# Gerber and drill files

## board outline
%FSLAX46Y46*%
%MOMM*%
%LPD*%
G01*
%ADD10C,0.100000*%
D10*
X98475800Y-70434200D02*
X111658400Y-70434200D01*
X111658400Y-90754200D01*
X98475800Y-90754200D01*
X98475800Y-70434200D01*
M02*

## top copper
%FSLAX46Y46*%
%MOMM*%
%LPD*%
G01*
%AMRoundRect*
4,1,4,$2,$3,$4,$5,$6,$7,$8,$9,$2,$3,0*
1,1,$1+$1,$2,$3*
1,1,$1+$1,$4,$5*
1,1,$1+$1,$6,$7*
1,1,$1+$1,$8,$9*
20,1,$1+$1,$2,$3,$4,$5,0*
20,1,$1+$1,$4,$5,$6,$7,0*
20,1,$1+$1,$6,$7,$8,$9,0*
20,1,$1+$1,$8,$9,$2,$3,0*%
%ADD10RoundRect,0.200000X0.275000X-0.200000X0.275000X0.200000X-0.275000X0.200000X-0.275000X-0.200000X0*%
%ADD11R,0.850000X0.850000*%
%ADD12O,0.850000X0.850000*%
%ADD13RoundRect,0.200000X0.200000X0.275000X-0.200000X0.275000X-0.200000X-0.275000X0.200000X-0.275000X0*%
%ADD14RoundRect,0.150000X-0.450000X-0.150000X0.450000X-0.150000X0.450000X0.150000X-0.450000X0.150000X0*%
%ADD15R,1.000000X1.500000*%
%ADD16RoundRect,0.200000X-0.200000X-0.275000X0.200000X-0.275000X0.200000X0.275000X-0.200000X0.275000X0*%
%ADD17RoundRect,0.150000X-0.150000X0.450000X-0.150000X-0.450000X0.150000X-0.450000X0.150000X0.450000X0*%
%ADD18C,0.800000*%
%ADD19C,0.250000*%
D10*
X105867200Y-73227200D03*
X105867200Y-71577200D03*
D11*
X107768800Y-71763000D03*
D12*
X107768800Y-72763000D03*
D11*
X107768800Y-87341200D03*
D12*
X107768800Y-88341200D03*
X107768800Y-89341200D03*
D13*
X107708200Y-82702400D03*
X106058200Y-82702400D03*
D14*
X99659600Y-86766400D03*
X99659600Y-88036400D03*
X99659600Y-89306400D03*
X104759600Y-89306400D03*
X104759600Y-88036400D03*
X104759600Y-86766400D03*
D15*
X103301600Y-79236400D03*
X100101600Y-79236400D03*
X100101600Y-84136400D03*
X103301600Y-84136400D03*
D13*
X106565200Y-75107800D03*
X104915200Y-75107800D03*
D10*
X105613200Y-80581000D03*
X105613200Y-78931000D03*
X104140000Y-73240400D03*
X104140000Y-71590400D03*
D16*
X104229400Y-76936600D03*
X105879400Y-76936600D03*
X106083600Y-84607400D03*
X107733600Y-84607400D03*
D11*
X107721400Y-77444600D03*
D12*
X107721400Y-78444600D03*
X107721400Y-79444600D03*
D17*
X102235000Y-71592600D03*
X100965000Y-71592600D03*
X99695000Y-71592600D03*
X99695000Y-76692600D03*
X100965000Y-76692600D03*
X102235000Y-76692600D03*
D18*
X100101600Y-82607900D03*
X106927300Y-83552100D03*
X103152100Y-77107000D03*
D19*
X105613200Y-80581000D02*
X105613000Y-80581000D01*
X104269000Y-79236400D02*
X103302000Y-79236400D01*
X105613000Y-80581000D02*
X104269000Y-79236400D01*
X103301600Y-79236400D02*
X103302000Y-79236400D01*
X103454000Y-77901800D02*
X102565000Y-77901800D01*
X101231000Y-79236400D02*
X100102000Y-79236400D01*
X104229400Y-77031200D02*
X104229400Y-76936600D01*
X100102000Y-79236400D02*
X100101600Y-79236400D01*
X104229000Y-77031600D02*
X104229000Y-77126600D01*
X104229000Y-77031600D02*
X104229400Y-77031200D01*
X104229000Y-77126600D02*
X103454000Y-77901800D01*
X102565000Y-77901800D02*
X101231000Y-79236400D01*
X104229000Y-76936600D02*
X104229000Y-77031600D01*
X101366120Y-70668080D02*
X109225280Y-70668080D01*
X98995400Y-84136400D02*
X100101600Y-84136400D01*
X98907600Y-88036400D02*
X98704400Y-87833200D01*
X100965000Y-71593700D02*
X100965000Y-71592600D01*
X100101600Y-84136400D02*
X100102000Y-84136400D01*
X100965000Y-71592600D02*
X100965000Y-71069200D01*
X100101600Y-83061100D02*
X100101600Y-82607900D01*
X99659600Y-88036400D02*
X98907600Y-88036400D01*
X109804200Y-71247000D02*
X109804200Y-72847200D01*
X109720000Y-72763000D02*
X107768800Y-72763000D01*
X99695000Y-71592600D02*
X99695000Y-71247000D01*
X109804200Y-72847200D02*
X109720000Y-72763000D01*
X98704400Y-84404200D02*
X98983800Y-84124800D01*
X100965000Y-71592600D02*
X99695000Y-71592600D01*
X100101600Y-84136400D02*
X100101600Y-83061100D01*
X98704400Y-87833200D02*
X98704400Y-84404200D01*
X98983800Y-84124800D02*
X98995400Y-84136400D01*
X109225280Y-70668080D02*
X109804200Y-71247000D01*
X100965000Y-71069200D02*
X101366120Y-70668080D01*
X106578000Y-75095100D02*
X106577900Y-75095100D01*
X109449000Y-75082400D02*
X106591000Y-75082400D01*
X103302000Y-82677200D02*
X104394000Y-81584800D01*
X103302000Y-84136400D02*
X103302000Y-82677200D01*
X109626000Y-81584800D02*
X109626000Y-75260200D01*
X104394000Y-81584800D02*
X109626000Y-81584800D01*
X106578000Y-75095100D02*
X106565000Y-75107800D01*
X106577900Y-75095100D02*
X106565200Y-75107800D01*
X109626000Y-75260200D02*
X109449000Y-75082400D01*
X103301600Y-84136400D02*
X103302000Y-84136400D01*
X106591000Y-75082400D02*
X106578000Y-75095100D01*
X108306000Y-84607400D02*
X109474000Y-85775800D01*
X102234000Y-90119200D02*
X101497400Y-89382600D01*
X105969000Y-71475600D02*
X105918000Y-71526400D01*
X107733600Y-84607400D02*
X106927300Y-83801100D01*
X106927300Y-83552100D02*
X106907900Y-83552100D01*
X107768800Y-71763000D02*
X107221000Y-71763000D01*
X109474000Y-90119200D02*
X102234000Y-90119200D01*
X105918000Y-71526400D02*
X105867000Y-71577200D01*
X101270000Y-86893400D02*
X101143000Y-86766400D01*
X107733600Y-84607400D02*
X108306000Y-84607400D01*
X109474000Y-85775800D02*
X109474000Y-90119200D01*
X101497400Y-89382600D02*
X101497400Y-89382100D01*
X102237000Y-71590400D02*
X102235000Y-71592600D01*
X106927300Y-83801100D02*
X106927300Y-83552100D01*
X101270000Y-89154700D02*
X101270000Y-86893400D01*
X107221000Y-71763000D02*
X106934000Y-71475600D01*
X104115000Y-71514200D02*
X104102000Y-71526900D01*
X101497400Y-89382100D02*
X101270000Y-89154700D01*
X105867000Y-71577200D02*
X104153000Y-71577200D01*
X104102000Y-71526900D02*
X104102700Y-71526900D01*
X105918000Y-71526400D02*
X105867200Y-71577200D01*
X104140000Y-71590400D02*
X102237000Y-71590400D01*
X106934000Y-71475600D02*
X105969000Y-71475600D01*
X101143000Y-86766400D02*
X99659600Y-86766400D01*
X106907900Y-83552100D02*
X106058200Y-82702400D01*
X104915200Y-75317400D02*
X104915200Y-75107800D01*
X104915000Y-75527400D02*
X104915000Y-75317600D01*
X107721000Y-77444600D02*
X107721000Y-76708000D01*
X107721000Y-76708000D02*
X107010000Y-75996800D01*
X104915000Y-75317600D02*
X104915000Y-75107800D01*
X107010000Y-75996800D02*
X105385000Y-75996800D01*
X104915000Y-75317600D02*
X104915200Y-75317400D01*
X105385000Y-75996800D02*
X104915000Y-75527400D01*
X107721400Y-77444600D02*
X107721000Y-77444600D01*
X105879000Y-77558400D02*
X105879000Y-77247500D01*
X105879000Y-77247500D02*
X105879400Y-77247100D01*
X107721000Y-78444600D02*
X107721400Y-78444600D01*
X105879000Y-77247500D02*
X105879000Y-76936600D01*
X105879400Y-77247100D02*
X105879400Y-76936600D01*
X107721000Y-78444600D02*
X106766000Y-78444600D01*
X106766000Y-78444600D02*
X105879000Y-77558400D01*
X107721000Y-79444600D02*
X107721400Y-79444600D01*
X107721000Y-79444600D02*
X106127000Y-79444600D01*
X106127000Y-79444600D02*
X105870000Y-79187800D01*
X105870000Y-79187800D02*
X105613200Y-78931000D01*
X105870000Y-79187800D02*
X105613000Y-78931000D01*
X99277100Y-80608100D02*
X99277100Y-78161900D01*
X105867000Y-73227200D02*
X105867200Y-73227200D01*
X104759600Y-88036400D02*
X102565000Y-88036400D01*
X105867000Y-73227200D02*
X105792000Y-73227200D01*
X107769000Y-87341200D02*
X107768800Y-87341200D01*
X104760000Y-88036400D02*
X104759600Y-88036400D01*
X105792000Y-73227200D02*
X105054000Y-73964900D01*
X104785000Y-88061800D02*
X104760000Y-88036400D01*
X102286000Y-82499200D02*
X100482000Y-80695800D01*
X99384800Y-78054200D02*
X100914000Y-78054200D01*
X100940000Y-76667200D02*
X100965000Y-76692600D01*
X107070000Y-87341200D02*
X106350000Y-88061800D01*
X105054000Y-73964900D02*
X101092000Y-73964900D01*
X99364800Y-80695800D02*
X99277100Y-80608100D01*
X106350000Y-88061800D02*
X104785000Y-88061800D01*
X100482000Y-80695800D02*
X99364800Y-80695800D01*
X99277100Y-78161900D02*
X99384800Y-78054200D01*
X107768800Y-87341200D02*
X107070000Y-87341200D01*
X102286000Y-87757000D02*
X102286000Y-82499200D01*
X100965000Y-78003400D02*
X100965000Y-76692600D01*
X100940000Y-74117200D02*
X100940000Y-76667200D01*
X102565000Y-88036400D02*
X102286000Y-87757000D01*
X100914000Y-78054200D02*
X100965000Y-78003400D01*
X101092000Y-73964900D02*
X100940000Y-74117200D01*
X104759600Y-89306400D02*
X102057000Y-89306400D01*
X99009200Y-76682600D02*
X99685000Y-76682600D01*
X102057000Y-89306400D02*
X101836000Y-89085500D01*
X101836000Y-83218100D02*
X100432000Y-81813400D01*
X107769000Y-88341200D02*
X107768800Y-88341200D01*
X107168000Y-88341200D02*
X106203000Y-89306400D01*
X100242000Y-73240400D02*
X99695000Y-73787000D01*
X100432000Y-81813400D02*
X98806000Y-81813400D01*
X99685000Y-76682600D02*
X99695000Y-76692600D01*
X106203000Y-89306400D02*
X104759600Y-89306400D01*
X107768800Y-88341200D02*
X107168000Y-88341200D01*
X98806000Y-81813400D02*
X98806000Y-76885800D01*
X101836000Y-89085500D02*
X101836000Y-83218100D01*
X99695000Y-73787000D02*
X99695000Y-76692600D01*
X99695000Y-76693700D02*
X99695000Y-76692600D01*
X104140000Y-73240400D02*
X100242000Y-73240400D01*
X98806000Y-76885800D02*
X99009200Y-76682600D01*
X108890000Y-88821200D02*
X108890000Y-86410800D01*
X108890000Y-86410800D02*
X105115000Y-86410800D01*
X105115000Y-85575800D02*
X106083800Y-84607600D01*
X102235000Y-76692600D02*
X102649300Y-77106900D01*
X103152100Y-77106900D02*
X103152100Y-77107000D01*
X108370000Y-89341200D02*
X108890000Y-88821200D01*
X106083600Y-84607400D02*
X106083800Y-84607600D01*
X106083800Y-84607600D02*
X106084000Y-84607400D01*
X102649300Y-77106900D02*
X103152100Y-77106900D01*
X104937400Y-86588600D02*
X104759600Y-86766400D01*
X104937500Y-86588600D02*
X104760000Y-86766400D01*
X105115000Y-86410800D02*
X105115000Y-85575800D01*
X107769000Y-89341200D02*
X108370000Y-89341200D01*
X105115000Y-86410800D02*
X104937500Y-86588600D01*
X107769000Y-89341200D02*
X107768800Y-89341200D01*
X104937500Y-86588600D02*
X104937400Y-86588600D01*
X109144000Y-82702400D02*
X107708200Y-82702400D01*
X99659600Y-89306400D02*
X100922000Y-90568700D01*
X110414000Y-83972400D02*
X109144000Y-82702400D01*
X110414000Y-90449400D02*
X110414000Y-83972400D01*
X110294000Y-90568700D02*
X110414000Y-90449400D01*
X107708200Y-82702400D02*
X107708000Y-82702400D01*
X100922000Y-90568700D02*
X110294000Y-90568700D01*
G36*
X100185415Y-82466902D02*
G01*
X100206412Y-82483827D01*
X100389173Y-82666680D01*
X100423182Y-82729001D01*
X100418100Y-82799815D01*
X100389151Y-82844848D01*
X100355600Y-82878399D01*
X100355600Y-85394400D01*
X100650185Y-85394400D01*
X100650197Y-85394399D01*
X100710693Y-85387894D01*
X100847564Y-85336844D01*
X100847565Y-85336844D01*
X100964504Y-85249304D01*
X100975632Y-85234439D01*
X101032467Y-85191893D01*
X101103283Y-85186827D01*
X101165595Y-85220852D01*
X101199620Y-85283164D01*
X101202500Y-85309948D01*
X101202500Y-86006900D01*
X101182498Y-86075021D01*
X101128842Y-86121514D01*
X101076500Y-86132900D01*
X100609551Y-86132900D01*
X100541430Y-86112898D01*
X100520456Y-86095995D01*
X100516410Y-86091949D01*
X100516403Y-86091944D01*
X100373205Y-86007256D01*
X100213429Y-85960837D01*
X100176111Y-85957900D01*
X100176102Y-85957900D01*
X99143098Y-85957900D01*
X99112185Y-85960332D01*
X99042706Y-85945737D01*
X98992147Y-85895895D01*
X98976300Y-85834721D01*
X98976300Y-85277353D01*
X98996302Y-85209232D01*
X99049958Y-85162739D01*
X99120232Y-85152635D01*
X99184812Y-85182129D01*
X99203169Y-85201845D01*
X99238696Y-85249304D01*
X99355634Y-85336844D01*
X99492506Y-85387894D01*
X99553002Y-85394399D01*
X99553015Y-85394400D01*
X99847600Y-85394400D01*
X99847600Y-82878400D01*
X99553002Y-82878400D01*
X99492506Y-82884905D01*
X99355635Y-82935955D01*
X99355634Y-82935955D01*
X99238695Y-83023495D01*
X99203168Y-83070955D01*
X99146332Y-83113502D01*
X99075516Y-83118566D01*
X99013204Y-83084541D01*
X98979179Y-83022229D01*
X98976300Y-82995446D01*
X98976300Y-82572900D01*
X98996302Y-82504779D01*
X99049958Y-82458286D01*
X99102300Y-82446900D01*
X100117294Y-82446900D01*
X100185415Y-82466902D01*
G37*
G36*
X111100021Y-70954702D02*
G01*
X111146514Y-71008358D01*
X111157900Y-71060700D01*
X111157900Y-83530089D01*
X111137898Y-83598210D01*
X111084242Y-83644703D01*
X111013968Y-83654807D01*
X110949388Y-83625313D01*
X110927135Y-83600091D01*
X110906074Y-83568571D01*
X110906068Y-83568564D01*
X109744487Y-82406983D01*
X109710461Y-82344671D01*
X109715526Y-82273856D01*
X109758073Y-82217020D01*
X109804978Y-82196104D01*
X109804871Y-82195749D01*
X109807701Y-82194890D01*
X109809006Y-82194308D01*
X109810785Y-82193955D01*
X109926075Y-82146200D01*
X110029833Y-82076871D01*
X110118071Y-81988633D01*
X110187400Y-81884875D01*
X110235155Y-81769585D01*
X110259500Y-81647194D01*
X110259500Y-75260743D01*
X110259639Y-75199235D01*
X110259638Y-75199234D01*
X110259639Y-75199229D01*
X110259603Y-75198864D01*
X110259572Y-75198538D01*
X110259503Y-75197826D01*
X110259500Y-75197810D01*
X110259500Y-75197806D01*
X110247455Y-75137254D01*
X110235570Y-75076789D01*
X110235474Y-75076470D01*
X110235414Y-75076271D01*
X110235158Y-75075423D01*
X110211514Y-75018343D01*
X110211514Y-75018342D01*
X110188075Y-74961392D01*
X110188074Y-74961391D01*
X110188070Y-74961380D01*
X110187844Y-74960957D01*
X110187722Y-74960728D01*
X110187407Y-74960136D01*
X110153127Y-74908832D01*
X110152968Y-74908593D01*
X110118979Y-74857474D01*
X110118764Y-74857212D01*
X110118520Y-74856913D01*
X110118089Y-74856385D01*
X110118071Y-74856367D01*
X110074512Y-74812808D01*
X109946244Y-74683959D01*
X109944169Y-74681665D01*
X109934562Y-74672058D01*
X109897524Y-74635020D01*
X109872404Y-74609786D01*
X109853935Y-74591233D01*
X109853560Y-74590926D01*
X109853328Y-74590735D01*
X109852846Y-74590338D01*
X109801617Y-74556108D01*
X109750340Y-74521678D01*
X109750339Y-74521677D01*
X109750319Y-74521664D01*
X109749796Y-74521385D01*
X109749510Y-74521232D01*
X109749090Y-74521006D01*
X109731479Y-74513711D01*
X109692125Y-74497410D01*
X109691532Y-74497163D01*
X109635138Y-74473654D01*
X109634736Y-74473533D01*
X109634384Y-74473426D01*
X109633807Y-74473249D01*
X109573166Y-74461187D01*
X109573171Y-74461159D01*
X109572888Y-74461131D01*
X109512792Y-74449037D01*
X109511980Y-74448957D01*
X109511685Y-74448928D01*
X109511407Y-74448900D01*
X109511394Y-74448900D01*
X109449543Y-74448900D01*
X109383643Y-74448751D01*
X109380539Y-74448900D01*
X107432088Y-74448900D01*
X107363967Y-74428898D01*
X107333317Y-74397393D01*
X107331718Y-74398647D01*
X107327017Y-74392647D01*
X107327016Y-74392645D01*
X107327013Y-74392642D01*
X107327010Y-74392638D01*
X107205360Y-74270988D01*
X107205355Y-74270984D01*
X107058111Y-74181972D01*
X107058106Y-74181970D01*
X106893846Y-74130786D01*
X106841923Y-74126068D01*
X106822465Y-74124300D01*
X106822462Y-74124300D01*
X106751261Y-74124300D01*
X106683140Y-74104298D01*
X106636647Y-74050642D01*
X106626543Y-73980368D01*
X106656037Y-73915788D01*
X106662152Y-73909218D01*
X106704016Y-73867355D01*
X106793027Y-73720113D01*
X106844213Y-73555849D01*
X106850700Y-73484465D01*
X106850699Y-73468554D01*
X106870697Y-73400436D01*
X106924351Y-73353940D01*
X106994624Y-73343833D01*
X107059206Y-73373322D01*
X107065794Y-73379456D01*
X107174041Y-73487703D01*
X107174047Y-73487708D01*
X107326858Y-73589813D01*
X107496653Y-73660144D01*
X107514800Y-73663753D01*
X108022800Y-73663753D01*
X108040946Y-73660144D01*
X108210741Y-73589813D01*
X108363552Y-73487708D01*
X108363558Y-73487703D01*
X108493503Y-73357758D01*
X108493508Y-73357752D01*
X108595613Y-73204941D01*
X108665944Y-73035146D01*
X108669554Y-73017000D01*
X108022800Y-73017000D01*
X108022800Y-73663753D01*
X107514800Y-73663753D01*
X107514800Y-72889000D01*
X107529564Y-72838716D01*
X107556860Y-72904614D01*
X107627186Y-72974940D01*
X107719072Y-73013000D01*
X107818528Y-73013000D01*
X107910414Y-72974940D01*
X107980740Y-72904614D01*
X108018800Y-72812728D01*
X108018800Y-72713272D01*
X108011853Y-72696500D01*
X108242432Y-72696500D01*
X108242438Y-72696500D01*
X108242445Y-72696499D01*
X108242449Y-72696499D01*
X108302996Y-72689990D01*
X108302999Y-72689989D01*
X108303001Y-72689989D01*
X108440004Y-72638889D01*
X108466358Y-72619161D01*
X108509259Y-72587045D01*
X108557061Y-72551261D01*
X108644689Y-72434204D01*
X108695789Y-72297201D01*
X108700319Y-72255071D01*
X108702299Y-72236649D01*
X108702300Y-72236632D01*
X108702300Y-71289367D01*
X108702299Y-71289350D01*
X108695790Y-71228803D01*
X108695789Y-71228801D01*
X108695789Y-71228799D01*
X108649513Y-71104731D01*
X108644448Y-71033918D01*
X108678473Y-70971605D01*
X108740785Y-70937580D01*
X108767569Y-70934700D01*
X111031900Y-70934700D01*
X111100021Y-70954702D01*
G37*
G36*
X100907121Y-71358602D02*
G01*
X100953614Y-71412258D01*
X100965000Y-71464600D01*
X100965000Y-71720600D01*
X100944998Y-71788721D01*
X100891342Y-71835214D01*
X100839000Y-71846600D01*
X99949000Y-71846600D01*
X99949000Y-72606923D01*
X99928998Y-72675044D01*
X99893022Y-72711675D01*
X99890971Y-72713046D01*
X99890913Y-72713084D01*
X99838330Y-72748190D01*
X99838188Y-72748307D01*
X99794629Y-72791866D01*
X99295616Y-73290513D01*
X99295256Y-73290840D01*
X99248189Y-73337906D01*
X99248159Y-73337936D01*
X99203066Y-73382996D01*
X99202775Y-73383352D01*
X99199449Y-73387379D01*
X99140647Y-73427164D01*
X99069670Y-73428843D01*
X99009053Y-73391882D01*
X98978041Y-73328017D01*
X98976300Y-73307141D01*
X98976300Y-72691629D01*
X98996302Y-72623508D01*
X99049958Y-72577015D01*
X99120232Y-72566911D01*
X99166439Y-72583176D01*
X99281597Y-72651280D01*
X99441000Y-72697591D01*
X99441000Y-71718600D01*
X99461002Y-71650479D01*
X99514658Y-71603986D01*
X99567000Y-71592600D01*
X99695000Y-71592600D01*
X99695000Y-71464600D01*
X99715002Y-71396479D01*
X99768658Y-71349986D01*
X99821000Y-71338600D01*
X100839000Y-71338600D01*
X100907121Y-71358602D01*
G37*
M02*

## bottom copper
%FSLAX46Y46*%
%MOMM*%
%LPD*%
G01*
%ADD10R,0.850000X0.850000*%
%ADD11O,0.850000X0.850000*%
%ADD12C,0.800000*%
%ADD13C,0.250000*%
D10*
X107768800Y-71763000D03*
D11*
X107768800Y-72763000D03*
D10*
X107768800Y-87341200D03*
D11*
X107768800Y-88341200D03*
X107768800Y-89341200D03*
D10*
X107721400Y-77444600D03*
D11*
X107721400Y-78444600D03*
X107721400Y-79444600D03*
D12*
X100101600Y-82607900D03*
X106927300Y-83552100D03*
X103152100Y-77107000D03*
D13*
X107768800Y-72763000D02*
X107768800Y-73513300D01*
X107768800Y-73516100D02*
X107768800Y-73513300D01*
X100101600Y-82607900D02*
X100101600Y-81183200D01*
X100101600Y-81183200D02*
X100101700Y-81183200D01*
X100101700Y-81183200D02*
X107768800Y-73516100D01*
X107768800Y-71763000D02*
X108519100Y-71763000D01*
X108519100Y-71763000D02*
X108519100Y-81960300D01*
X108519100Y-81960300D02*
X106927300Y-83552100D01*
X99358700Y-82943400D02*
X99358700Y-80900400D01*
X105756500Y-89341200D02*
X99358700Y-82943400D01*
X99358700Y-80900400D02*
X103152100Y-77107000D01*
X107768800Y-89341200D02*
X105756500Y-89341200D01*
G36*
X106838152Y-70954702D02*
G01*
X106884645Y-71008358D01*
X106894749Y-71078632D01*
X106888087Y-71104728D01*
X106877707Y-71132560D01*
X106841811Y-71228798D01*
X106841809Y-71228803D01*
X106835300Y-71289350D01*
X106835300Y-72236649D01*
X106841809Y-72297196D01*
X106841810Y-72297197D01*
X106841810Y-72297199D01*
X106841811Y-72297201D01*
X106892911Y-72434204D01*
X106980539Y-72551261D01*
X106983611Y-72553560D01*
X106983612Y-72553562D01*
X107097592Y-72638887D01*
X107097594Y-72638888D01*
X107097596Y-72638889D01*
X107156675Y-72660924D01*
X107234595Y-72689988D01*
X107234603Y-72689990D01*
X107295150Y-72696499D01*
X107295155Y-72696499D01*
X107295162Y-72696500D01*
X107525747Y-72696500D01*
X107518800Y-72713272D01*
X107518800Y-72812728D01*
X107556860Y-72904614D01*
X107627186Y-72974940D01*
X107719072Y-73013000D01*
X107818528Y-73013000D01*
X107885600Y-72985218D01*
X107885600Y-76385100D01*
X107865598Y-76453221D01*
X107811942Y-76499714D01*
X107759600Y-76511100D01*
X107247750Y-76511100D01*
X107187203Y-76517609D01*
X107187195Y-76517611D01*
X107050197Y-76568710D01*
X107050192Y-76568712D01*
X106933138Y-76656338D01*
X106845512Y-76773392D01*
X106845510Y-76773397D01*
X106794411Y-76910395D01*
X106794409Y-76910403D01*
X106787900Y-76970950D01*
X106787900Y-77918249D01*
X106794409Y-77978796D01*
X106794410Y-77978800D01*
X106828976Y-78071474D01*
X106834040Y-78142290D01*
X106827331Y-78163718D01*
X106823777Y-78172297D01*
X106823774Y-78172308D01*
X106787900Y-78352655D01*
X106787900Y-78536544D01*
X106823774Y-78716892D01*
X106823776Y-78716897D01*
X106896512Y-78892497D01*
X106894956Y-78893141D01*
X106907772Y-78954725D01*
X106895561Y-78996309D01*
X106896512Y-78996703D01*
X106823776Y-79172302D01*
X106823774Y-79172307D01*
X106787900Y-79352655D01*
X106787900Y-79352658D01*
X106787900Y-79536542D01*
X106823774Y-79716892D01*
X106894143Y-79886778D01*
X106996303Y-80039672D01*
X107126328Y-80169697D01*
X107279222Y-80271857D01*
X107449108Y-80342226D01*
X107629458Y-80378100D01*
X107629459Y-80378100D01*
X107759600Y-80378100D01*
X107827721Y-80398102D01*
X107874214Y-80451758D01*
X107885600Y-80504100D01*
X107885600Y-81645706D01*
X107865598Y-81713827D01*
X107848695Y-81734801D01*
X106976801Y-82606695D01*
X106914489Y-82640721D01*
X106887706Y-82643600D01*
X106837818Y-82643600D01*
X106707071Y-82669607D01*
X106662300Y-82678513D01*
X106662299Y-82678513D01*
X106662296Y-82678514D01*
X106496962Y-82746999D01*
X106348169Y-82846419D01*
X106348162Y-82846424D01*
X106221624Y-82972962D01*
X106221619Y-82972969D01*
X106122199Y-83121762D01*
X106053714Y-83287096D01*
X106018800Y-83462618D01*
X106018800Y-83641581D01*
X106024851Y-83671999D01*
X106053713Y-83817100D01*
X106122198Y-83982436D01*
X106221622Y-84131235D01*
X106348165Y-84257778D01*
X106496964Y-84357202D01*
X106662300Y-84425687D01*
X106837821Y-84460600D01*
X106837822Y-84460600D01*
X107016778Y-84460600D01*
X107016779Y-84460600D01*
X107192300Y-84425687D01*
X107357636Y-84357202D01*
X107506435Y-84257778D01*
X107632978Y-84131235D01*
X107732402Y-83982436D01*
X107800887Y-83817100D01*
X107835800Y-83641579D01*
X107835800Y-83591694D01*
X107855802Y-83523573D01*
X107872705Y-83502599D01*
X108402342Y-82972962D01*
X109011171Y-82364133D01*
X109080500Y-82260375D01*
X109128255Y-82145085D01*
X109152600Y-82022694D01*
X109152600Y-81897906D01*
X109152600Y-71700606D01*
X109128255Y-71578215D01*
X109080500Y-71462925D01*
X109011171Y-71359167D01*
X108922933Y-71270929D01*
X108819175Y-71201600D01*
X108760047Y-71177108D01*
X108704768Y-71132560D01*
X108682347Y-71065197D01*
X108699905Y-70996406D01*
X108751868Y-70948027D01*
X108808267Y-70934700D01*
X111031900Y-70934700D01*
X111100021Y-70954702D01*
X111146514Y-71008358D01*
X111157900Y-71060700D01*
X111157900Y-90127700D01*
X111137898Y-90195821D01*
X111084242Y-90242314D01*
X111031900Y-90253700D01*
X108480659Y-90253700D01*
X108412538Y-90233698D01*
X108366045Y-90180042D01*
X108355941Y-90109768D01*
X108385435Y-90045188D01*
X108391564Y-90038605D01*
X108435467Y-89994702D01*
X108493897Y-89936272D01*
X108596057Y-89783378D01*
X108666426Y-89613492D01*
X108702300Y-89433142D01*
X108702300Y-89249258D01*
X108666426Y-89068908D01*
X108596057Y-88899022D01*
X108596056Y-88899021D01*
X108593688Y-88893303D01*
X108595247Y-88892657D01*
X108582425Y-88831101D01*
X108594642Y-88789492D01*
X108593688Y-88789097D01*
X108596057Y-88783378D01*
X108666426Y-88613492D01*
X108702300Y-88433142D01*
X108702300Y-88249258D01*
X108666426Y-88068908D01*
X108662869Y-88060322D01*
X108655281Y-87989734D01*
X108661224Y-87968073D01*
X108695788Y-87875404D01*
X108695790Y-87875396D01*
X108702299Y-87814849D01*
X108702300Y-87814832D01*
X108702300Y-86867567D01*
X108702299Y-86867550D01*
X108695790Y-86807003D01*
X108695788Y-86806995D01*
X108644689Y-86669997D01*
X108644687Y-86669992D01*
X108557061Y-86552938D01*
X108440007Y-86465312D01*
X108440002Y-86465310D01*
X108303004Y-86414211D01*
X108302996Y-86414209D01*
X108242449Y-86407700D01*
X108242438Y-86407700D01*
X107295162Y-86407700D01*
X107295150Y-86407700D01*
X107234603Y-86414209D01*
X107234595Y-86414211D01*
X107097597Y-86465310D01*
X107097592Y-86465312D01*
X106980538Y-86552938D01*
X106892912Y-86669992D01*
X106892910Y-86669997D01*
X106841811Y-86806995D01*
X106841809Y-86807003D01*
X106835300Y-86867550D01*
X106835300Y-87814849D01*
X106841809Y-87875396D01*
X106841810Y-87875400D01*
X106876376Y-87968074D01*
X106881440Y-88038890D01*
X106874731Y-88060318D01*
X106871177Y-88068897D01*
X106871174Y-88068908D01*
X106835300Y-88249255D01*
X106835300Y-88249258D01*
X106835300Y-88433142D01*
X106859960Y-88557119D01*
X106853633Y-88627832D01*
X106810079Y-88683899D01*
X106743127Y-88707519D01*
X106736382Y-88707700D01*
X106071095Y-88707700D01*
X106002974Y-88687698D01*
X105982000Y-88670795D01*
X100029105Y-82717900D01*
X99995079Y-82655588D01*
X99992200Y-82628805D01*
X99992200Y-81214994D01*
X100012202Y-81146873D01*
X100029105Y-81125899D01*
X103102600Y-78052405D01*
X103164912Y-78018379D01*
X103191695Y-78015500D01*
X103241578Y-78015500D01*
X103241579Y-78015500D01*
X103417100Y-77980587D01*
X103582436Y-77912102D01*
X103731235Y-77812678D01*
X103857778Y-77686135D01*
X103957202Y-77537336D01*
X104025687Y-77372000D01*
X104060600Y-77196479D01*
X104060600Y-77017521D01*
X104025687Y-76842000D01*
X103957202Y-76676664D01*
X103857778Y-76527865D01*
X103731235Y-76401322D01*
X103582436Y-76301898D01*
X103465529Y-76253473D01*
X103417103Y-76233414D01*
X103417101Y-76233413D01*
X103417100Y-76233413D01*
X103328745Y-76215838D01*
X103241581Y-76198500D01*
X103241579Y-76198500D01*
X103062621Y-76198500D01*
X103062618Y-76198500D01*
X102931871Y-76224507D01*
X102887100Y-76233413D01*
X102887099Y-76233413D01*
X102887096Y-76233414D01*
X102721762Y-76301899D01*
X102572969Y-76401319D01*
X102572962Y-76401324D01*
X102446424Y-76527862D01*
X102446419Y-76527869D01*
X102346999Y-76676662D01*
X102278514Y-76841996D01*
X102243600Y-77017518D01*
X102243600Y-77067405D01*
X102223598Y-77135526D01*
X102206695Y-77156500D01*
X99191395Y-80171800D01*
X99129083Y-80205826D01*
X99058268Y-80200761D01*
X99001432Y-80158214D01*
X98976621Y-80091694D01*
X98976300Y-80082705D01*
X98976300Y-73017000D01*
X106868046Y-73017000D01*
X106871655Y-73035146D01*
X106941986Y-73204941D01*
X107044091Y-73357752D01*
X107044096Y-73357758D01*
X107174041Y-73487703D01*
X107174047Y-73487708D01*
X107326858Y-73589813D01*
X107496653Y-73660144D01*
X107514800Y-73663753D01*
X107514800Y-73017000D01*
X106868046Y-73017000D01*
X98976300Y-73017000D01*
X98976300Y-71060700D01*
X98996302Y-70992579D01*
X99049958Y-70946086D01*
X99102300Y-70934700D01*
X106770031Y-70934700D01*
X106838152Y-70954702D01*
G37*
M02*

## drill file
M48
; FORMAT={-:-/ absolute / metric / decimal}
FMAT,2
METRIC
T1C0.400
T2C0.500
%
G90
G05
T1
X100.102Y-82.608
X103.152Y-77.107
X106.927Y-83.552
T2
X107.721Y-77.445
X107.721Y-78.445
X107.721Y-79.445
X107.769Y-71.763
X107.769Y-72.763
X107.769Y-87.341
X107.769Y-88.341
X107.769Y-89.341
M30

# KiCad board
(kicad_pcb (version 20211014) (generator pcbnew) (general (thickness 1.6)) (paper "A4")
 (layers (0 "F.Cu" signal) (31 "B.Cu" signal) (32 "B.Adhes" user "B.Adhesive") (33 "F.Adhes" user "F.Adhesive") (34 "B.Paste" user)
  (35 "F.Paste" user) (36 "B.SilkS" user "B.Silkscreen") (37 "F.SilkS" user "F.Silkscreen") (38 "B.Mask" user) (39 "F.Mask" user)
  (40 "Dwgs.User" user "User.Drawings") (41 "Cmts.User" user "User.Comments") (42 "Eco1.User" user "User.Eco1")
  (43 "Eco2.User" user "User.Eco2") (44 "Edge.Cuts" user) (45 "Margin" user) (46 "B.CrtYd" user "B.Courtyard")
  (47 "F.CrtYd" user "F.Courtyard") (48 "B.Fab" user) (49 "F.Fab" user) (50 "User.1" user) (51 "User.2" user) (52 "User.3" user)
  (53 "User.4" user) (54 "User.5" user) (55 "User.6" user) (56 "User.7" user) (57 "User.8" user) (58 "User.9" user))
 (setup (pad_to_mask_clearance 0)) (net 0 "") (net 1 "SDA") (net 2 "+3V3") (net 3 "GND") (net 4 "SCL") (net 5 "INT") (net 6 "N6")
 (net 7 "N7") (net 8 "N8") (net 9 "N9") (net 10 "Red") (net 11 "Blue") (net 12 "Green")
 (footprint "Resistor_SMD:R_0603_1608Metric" (layer "F.Cu") (at 105.8672 72.4022 90)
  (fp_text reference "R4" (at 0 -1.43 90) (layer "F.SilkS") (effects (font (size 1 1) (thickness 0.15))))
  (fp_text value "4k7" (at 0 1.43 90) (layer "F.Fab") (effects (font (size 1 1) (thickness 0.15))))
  (pad "1" smd roundrect (at -0.825 0 90) (size 0.8 0.95) (layers "F.Cu" "F.Paste" "F.Mask") (roundrect_rratio 0.25) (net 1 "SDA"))
  (pad "2" smd roundrect (at 0.825 0 90) (size 0.8 0.95) (layers "F.Cu" "F.Paste" "F.Mask") (roundrect_rratio 0.25) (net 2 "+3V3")))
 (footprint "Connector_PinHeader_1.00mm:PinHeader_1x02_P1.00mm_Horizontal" (layer "F.Cu") (at 107.7688 71.763)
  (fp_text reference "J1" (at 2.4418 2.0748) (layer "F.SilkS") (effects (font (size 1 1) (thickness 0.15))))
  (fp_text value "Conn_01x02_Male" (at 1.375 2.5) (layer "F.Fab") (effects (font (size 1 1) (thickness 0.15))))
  (pad "1" thru_hole rect (at 0 0) (size 0.85 0.85) (drill 0.5) (layers *.Cu *.Mask) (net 2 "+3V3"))
  (pad "2" thru_hole oval (at 0 1) (size 0.85 0.85) (drill 0.5) (layers *.Cu *.Mask) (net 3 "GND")))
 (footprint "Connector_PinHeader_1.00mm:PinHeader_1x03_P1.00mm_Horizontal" (layer "F.Cu") (at 107.7688 87.3412)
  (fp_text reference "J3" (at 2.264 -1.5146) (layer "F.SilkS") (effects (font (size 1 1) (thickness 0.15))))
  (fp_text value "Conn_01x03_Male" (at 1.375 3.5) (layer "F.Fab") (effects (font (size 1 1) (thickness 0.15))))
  (pad "1" thru_hole rect (at 0 0) (size 0.85 0.85) (drill 0.5) (layers *.Cu *.Mask) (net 1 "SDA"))
  (pad "2" thru_hole oval (at 0 1) (size 0.85 0.85) (drill 0.5) (layers *.Cu *.Mask) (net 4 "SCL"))
  (pad "3" thru_hole oval (at 0 2) (size 0.85 0.85) (drill 0.5) (layers *.Cu *.Mask) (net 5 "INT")))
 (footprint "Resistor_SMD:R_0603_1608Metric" (layer "F.Cu") (at 106.8832 82.7024 180)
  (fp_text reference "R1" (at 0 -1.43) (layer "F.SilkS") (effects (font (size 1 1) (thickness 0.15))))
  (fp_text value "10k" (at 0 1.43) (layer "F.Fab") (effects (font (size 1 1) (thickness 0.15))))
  (pad "1" smd roundrect (at -0.825 0 180) (size 0.8 0.95) (layers "F.Cu" "F.Paste" "F.Mask") (roundrect_rratio 0.25) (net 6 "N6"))
  (pad "2" smd roundrect (at 0.825 0 180) (size 0.8 0.95) (layers "F.Cu" "F.Paste" "F.Mask") (roundrect_rratio 0.25) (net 2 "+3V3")))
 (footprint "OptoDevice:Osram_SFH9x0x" (layer "F.Cu") (at 102.2096 88.0364)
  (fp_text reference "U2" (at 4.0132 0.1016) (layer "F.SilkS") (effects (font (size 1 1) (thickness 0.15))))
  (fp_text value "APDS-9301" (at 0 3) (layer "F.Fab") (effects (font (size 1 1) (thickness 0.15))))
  (pad "1" smd roundrect (at -2.55 -1.27) (size 1.2 0.6) (layers "F.Cu" "F.Paste" "F.Mask") (roundrect_rratio 0.25) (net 2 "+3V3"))
  (pad "2" smd roundrect (at -2.55 0) (size 1.2 0.6) (layers "F.Cu" "F.Paste" "F.Mask") (roundrect_rratio 0.25) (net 3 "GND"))
  (pad "3" smd roundrect (at -2.55 1.27) (size 1.2 0.6) (layers "F.Cu" "F.Paste" "F.Mask") (roundrect_rratio 0.25) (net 6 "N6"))
  (pad "4" smd roundrect (at 2.55 1.27) (size 1.2 0.6) (layers "F.Cu" "F.Paste" "F.Mask") (roundrect_rratio 0.25) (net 4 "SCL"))
  (pad "5" smd roundrect (at 2.55 0) (size 1.2 0.6) (layers "F.Cu" "F.Paste" "F.Mask") (roundrect_rratio 0.25) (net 1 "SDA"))
  (pad "6" smd roundrect (at 2.55 -1.27) (size 1.2 0.6) (layers "F.Cu" "F.Paste" "F.Mask") (roundrect_rratio 0.25) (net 5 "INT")))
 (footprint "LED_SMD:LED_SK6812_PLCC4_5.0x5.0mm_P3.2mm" (layer "F.Cu") (at 101.7016 81.6864 90)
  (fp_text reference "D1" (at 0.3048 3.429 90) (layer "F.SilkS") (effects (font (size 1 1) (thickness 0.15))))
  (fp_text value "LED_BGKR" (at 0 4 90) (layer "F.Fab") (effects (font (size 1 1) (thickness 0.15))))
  (pad "1" smd rect (at 2.45 1.6 90) (size 1.5 1) (layers "F.Cu" "F.Paste" "F.Mask") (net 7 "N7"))
  (pad "2" smd rect (at 2.45 -1.6 90) (size 1.5 1) (layers "F.Cu" "F.Paste" "F.Mask") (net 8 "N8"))
  (pad "3" smd rect (at -2.45 -1.6 90) (size 1.5 1) (layers "F.Cu" "F.Paste" "F.Mask") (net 3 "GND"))
  (pad "4" smd rect (at -2.45 1.6 90) (size 1.5 1) (layers "F.Cu" "F.Paste" "F.Mask") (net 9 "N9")))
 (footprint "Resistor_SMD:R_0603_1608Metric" (layer "F.Cu") (at 105.7402 75.1078 180)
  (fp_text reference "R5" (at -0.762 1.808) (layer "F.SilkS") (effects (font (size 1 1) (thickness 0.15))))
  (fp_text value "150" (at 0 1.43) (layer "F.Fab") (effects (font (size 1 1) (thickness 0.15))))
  (pad "1" smd roundrect (at -0.825 0 180) (size 0.8 0.95) (layers "F.Cu" "F.Paste" "F.Mask") (roundrect_rratio 0.25) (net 9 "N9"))
  (pad "2" smd roundrect (at 0.825 0 180) (size 0.8 0.95) (layers "F.Cu" "F.Paste" "F.Mask") (roundrect_rratio 0.25) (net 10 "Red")))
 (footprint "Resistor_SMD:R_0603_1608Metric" (layer "F.Cu") (at 105.6132 79.756 90)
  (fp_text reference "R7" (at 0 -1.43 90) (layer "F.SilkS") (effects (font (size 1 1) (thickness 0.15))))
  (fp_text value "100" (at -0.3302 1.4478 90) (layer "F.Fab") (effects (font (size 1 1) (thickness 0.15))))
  (pad "1" smd roundrect (at -0.825 0 90) (size 0.8 0.95) (layers "F.Cu" "F.Paste" "F.Mask") (roundrect_rratio 0.25) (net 7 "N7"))
  (pad "2" smd roundrect (at 0.825 0 90) (size 0.8 0.95) (layers "F.Cu" "F.Paste" "F.Mask") (roundrect_rratio 0.25) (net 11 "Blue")))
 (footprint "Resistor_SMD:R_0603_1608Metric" (layer "F.Cu") (at 104.14 72.4154 90)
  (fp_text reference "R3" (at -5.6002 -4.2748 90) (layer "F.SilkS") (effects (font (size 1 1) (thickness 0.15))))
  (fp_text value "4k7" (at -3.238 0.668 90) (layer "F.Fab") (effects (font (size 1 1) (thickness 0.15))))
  (pad "1" smd roundrect (at -0.825 0 90) (size 0.8 0.95) (layers "F.Cu" "F.Paste" "F.Mask") (roundrect_rratio 0.25) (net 4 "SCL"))
  (pad "2" smd roundrect (at 0.825 0 90) (size 0.8 0.95) (layers "F.Cu" "F.Paste" "F.Mask") (roundrect_rratio 0.25) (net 2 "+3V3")))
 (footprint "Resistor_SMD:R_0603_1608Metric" (layer "F.Cu") (at 105.0544 76.9366)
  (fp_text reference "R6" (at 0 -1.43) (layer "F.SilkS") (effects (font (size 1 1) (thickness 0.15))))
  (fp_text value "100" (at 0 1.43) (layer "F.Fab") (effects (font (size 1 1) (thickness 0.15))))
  (pad "1" smd roundrect (at -0.825 0) (size 0.8 0.95) (layers "F.Cu" "F.Paste" "F.Mask") (roundrect_rratio 0.25) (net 8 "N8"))
  (pad "2" smd roundrect (at 0.825 0) (size 0.8 0.95) (layers "F.Cu" "F.Paste" "F.Mask") (roundrect_rratio 0.25) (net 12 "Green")))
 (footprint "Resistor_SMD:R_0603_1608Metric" (layer "F.Cu") (at 106.9086 84.6074)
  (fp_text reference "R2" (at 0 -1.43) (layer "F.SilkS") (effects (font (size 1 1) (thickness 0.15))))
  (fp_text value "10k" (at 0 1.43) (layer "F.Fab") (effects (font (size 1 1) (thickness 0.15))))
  (pad "1" smd roundrect (at -0.825 0) (size 0.8 0.95) (layers "F.Cu" "F.Paste" "F.Mask") (roundrect_rratio 0.25) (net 5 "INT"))
  (pad "2" smd roundrect (at 0.825 0) (size 0.8 0.95) (layers "F.Cu" "F.Paste" "F.Mask") (roundrect_rratio 0.25) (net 2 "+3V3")))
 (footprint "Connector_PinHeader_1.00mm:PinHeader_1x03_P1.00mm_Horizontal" (layer "F.Cu") (at 107.7214 77.4446)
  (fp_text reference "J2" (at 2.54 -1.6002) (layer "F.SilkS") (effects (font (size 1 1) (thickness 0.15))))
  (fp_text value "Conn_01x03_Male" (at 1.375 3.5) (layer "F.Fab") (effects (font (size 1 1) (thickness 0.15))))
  (pad "1" thru_hole rect (at 0 0) (size 0.85 0.85) (drill 0.5) (layers *.Cu *.Mask) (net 10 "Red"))
  (pad "2" thru_hole oval (at 0 1) (size 0.85 0.85) (drill 0.5) (layers *.Cu *.Mask) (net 12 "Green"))
  (pad "3" thru_hole oval (at 0 2) (size 0.85 0.85) (drill 0.5) (layers *.Cu *.Mask) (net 11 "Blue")))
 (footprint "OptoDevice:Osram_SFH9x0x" (layer "F.Cu") (at 100.965 74.1426 -90)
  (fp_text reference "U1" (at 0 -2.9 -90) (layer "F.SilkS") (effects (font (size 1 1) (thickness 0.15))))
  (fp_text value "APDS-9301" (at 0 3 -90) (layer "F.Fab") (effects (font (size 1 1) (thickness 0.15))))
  (pad "1" smd roundrect (at -2.55 -1.27 270) (size 1.2 0.6) (layers "F.Cu" "F.Paste" "F.Mask") (roundrect_rratio 0.25) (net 2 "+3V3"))
  (pad "2" smd roundrect (at -2.55 0 270) (size 1.2 0.6) (layers "F.Cu" "F.Paste" "F.Mask") (roundrect_rratio 0.25) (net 3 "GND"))
  (pad "3" smd roundrect (at -2.55 1.27 270) (size 1.2 0.6) (layers "F.Cu" "F.Paste" "F.Mask") (roundrect_rratio 0.25) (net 3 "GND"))
  (pad "4" smd roundrect (at 2.55 1.27 270) (size 1.2 0.6) (layers "F.Cu" "F.Paste" "F.Mask") (roundrect_rratio 0.25) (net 4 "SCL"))
  (pad "5" smd roundrect (at 2.55 0 270) (size 1.2 0.6) (layers "F.Cu" "F.Paste" "F.Mask") (roundrect_rratio 0.25) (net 1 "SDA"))
  (pad "6" smd roundrect (at 2.55 -1.27 270) (size 1.2 0.6) (layers "F.Cu" "F.Paste" "F.Mask") (roundrect_rratio 0.25) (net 5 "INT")))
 (gr_rect (start 98.4758 70.4342) (end 111.6584 90.7542) (layer "Edge.Cuts") (width 0.1) (fill none))
 (segment (start 105.6132 80.581) (end 105.613 80.581) (width 0.25) (layer "F.Cu") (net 7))
 (segment (start 104.269 79.2364) (end 103.302 79.2364) (width 0.25) (layer "F.Cu") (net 7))
 (segment (start 105.613 80.581) (end 104.269 79.2364) (width 0.25) (layer "F.Cu") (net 7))
 (segment (start 103.3016 79.2364) (end 103.302 79.2364) (width 0.25) (layer "F.Cu") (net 7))
 (segment (start 103.454 77.9018) (end 102.565 77.9018) (width 0.25) (layer "F.Cu") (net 8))
 (segment (start 101.231 79.2364) (end 100.102 79.2364) (width 0.25) (layer "F.Cu") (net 8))
 (segment (start 104.2294 77.0312) (end 104.2294 76.9366) (width 0.25) (layer "F.Cu") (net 8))
 (segment (start 100.102 79.2364) (end 100.1016 79.2364) (width 0.25) (layer "F.Cu") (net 8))
 (segment (start 104.229 77.0316) (end 104.229 77.1266) (width 0.25) (layer "F.Cu") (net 8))
 (segment (start 104.229 77.0316) (end 104.2294 77.0312) (width 0.25) (layer "F.Cu") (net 8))
 (segment (start 104.229 77.1266) (end 103.454 77.9018) (width 0.25) (layer "F.Cu") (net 8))
 (segment (start 102.565 77.9018) (end 101.231 79.2364) (width 0.25) (layer "F.Cu") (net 8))
 (segment (start 104.229 76.9366) (end 104.229 77.0316) (width 0.25) (layer "F.Cu") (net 8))
 (segment (start 101.36612 70.66808) (end 109.22528 70.66808) (width 0.25) (layer "F.Cu") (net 3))
 (segment (start 98.9954 84.1364) (end 100.1016 84.1364) (width 0.25) (layer "F.Cu") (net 3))
 (segment (start 98.9076 88.0364) (end 98.7044 87.8332) (width 0.25) (layer "F.Cu") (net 3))
 (segment (start 100.965 71.5937) (end 100.965 71.5926) (width 0.25) (layer "F.Cu") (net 3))
 (segment (start 100.1016 84.1364) (end 100.102 84.1364) (width 0.25) (layer "F.Cu") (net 3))
 (segment (start 100.965 71.5926) (end 100.965 71.0692) (width 0.25) (layer "F.Cu") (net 3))
 (segment (start 100.1016 83.0611) (end 100.1016 82.6079) (width 0.25) (layer "F.Cu") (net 3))
 (segment (start 99.6596 88.0364) (end 98.9076 88.0364) (width 0.25) (layer "F.Cu") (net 3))
 (segment (start 109.8042 71.247) (end 109.8042 72.8472) (width 0.25) (layer "F.Cu") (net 3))
 (segment (start 109.72 72.763) (end 107.7688 72.763) (width 0.25) (layer "F.Cu") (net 3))
 (segment (start 99.695 71.5926) (end 99.695 71.247) (width 0.25) (layer "F.Cu") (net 3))
 (segment (start 109.8042 72.8472) (end 109.72 72.763) (width 0.25) (layer "F.Cu") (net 3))
 (segment (start 98.7044 84.4042) (end 98.9838 84.1248) (width 0.25) (layer "F.Cu") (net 3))
 (segment (start 100.965 71.5926) (end 99.695 71.5926) (width 0.25) (layer "F.Cu") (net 3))
 (segment (start 100.1016 84.1364) (end 100.1016 83.0611) (width 0.25) (layer "F.Cu") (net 3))
 (segment (start 98.7044 87.8332) (end 98.7044 84.4042) (width 0.25) (layer "F.Cu") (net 3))
 (segment (start 98.9838 84.1248) (end 98.9954 84.1364) (width 0.25) (layer "F.Cu") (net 3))
 (segment (start 109.22528 70.66808) (end 109.8042 71.247) (width 0.25) (layer "F.Cu") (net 3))
 (segment (start 100.965 71.0692) (end 101.36612 70.66808) (width 0.25) (layer "F.Cu") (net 3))
 (via (at 100.1016 82.6079) (size 0.8) (drill 0.4) (layers "F.Cu" "B.Cu") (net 3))
 (segment (start 107.7688 72.763) (end 107.7688 73.5133) (width 0.25) (layer "B.Cu") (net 3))
 (segment (start 107.7688 73.5161) (end 107.7688 73.5133) (width 0.25) (layer "B.Cu") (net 3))
 (segment (start 100.1016 82.6079) (end 100.1016 81.1832) (width 0.25) (layer "B.Cu") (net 3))
 (segment (start 100.1016 81.1832) (end 100.1017 81.1832) (width 0.25) (layer "B.Cu") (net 3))
 (segment (start 100.1017 81.1832) (end 107.7688 73.5161) (width 0.25) (layer "B.Cu") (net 3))
 (segment (start 106.578 75.0951) (end 106.5779 75.0951) (width 0.25) (layer "F.Cu") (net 9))
 (segment (start 109.449 75.0824) (end 106.591 75.0824) (width 0.25) (layer "F.Cu") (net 9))
 (segment (start 103.302 82.6772) (end 104.394 81.5848) (width 0.25) (layer "F.Cu") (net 9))
 (segment (start 103.302 84.1364) (end 103.302 82.6772) (width 0.25) (layer "F.Cu") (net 9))
 (segment (start 109.626 81.5848) (end 109.626 75.2602) (width 0.25) (layer "F.Cu") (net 9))
 (segment (start 104.394 81.5848) (end 109.626 81.5848) (width 0.25) (layer "F.Cu") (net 9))
 (segment (start 106.578 75.0951) (end 106.565 75.1078) (width 0.25) (layer "F.Cu") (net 9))
 (segment (start 106.5779 75.0951) (end 106.5652 75.1078) (width 0.25) (layer "F.Cu") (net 9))
 (segment (start 109.626 75.2602) (end 109.449 75.0824) (width 0.25) (layer "F.Cu") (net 9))
 (segment (start 103.3016 84.1364) (end 103.302 84.1364) (width 0.25) (layer "F.Cu") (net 9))
 (segment (start 106.591 75.0824) (end 106.578 75.0951) (width 0.25) (layer "F.Cu") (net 9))
 (segment (start 108.306 84.6074) (end 109.474 85.7758) (width 0.25) (layer "F.Cu") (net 2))
 (segment (start 102.234 90.1192) (end 101.4974 89.3826) (width 0.25) (layer "F.Cu") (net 2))
 (segment (start 105.969 71.4756) (end 105.918 71.5264) (width 0.25) (layer "F.Cu") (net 2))
 (segment (start 107.7336 84.6074) (end 106.9273 83.8011) (width 0.25) (layer "F.Cu") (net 2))
 (segment (start 106.9273 83.5521) (end 106.9079 83.5521) (width 0.25) (layer "F.Cu") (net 2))
 (segment (start 107.7688 71.763) (end 107.221 71.763) (width 0.25) (layer "F.Cu") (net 2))
 (segment (start 109.474 90.1192) (end 102.234 90.1192) (width 0.25) (layer "F.Cu") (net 2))
 (segment (start 105.918 71.5264) (end 105.867 71.5772) (width 0.25) (layer "F.Cu") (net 2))
 (segment (start 101.27 86.8934) (end 101.143 86.7664) (width 0.25) (layer "F.Cu") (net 2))
 (segment (start 107.7336 84.6074) (end 108.306 84.6074) (width 0.25) (layer "F.Cu") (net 2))
 (segment (start 109.474 85.7758) (end 109.474 90.1192) (width 0.25) (layer "F.Cu") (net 2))
 (segment (start 101.4974 89.3826) (end 101.4974 89.3821) (width 0.25) (layer "F.Cu") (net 2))
 (segment (start 102.237 71.5904) (end 102.235 71.5926) (width 0.25) (layer "F.Cu") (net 2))
 (segment (start 106.9273 83.8011) (end 106.9273 83.5521) (width 0.25) (layer "F.Cu") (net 2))
 (segment (start 101.27 89.1547) (end 101.27 86.8934) (width 0.25) (layer "F.Cu") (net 2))
 (segment (start 107.221 71.763) (end 106.934 71.4756) (width 0.25) (layer "F.Cu") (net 2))
 (segment (start 104.115 71.5142) (end 104.102 71.5269) (width 0.25) (layer "F.Cu") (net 2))
 (segment (start 101.4974 89.3821) (end 101.27 89.1547) (width 0.25) (layer "F.Cu") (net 2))
 (segment (start 105.867 71.5772) (end 104.153 71.5772) (width 0.25) (layer "F.Cu") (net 2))
 (segment (start 104.102 71.5269) (end 104.1027 71.5269) (width 0.25) (layer "F.Cu") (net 2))
 (segment (start 105.918 71.5264) (end 105.8672 71.5772) (width 0.25) (layer "F.Cu") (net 2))
 (segment (start 104.14 71.5904) (end 102.237 71.5904) (width 0.25) (layer "F.Cu") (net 2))
 (segment (start 106.934 71.4756) (end 105.969 71.4756) (width 0.25) (layer "F.Cu") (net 2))
 (segment (start 101.143 86.7664) (end 99.6596 86.7664) (width 0.25) (layer "F.Cu") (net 2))
 (segment (start 106.9079 83.5521) (end 106.0582 82.7024) (width 0.25) (layer "F.Cu") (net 2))
 (via (at 106.9273 83.5521) (size 0.8) (drill 0.4) (layers "F.Cu" "B.Cu") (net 2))
 (segment (start 107.7688 71.763) (end 108.5191 71.763) (width 0.25) (layer "B.Cu") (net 2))
 (segment (start 108.5191 71.763) (end 108.5191 81.9603) (width 0.25) (layer "B.Cu") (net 2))
 (segment (start 108.5191 81.9603) (end 106.9273 83.5521) (width 0.25) (layer "B.Cu") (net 2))
 (segment (start 104.9152 75.3174) (end 104.9152 75.1078) (width 0.25) (layer "F.Cu") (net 10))
 (segment (start 104.915 75.5274) (end 104.915 75.3176) (width 0.25) (layer "F.Cu") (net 10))
 (segment (start 107.721 77.4446) (end 107.721 76.708) (width 0.25) (layer "F.Cu") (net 10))
 (segment (start 107.721 76.708) (end 107.01 75.9968) (width 0.25) (layer "F.Cu") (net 10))
 (segment (start 104.915 75.3176) (end 104.915 75.1078) (width 0.25) (layer "F.Cu") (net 10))
 (segment (start 107.01 75.9968) (end 105.385 75.9968) (width 0.25) (layer "F.Cu") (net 10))
 (segment (start 104.915 75.3176) (end 104.9152 75.3174) (width 0.25) (layer "F.Cu") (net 10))
 (segment (start 105.385 75.9968) (end 104.915 75.5274) (width 0.25) (layer "F.Cu") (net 10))
 (segment (start 107.7214 77.4446) (end 107.721 77.4446) (width 0.25) (layer "F.Cu") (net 10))
 (segment (start 105.879 77.5584) (end 105.879 77.2475) (width 0.25) (layer "F.Cu") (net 12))
 (segment (start 105.879 77.2475) (end 105.8794 77.2471) (width 0.25) (layer "F.Cu") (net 12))
 (segment (start 107.721 78.4446) (end 107.7214 78.4446) (width 0.25) (layer "F.Cu") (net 12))
 (segment (start 105.879 77.2475) (end 105.879 76.9366) (width 0.25) (layer "F.Cu") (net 12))
 (segment (start 105.8794 77.2471) (end 105.8794 76.9366) (width 0.25) (layer "F.Cu") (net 12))
 (segment (start 107.721 78.4446) (end 106.766 78.4446) (width 0.25) (layer "F.Cu") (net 12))
 (segment (start 106.766 78.4446) (end 105.879 77.5584) (width 0.25) (layer "F.Cu") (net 12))
 (segment (start 107.721 79.4446) (end 107.7214 79.4446) (width 0.25) (layer "F.Cu") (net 11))
 (segment (start 107.721 79.4446) (end 106.127 79.4446) (width 0.25) (layer "F.Cu") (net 11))
 (segment (start 106.127 79.4446) (end 105.87 79.1878) (width 0.25) (layer "F.Cu") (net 11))
 (segment (start 105.87 79.1878) (end 105.6132 78.931) (width 0.25) (layer "F.Cu") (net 11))
 (segment (start 105.87 79.1878) (end 105.613 78.931) (width 0.25) (layer "F.Cu") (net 11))
 (segment (start 99.2771 80.6081) (end 99.2771 78.1619) (width 0.25) (layer "F.Cu") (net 1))
 (segment (start 105.867 73.2272) (end 105.8672 73.2272) (width 0.25) (layer "F.Cu") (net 1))
 (segment (start 104.7596 88.0364) (end 102.565 88.0364) (width 0.25) (layer "F.Cu") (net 1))
 (segment (start 105.867 73.2272) (end 105.792 73.2272) (width 0.25) (layer "F.Cu") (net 1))
 (segment (start 107.769 87.3412) (end 107.7688 87.3412) (width 0.25) (layer "F.Cu") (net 1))
 (segment (start 104.76 88.0364) (end 104.7596 88.0364) (width 0.25) (layer "F.Cu") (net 1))
 (segment (start 105.792 73.2272) (end 105.054 73.9649) (width 0.25) (layer "F.Cu") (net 1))
 (segment (start 104.785 88.0618) (end 104.76 88.0364) (width 0.25) (layer "F.Cu") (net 1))
 (segment (start 102.286 82.4992) (end 100.482 80.6958) (width 0.25) (layer "F.Cu") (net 1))
 (segment (start 99.3848 78.0542) (end 100.914 78.0542) (width 0.25) (layer "F.Cu") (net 1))
 (segment (start 100.94 76.6672) (end 100.965 76.6926) (width 0.25) (layer "F.Cu") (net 1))
 (segment (start 107.07 87.3412) (end 106.35 88.0618) (width 0.25) (layer "F.Cu") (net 1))
 (segment (start 105.054 73.9649) (end 101.092 73.9649) (width 0.25) (layer "F.Cu") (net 1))
 (segment (start 99.3648 80.6958) (end 99.2771 80.6081) (width 0.25) (layer "F.Cu") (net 1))
 (segment (start 106.35 88.0618) (end 104.785 88.0618) (width 0.25) (layer "F.Cu") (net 1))
 (segment (start 100.482 80.6958) (end 99.3648 80.6958) (width 0.25) (layer "F.Cu") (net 1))
 (segment (start 99.2771 78.1619) (end 99.3848 78.0542) (width 0.25) (layer "F.Cu") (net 1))
 (segment (start 107.7688 87.3412) (end 107.07 87.3412) (width 0.25) (layer "F.Cu") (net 1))
 (segment (start 102.286 87.757) (end 102.286 82.4992) (width 0.25) (layer "F.Cu") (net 1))
 (segment (start 100.965 78.0034) (end 100.965 76.6926) (width 0.25) (layer "F.Cu") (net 1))
 (segment (start 100.94 74.1172) (end 100.94 76.6672) (width 0.25) (layer "F.Cu") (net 1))
 (segment (start 102.565 88.0364) (end 102.286 87.757) (width 0.25) (layer "F.Cu") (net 1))
 (segment (start 100.914 78.0542) (end 100.965 78.0034) (width 0.25) (layer "F.Cu") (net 1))
 (segment (start 101.092 73.9649) (end 100.94 74.1172) (width 0.25) (layer "F.Cu") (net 1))
 (segment (start 104.7596 89.3064) (end 102.057 89.3064) (width 0.25) (layer "F.Cu") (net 4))
 (segment (start 99.0092 76.6826) (end 99.685 76.6826) (width 0.25) (layer "F.Cu") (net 4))
 (segment (start 102.057 89.3064) (end 101.836 89.0855) (width 0.25) (layer "F.Cu") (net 4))
 (segment (start 101.836 83.2181) (end 100.432 81.8134) (width 0.25) (layer "F.Cu") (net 4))
 (segment (start 107.769 88.3412) (end 107.7688 88.3412) (width 0.25) (layer "F.Cu") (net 4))
 (segment (start 107.168 88.3412) (end 106.203 89.3064) (width 0.25) (layer "F.Cu") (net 4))
 (segment (start 100.242 73.2404) (end 99.695 73.787) (width 0.25) (layer "F.Cu") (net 4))
 (segment (start 100.432 81.8134) (end 98.806 81.8134) (width 0.25) (layer "F.Cu") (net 4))
 (segment (start 99.685 76.6826) (end 99.695 76.6926) (width 0.25) (layer "F.Cu") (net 4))
 (segment (start 106.203 89.3064) (end 104.7596 89.3064) (width 0.25) (layer "F.Cu") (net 4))
 (segment (start 107.7688 88.3412) (end 107.168 88.3412) (width 0.25) (layer "F.Cu") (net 4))
 (segment (start 98.806 81.8134) (end 98.806 76.8858) (width 0.25) (layer "F.Cu") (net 4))
 (segment (start 101.836 89.0855) (end 101.836 83.2181) (width 0.25) (layer "F.Cu") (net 4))
 (segment (start 99.695 73.787) (end 99.695 76.6926) (width 0.25) (layer "F.Cu") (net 4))
 (segment (start 99.695 76.6937) (end 99.695 76.6926) (width 0.25) (layer "F.Cu") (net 4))
 (segment (start 104.14 73.2404) (end 100.242 73.2404) (width 0.25) (layer "F.Cu") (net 4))
 (segment (start 98.806 76.8858) (end 99.0092 76.6826) (width 0.25) (layer "F.Cu") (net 4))
 (segment (start 108.89 88.8212) (end 108.89 86.4108) (width 0.25) (layer "F.Cu") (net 5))
 (segment (start 108.89 86.4108) (end 105.115 86.4108) (width 0.25) (layer "F.Cu") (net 5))
 (segment (start 105.115 85.5758) (end 106.0838 84.6076) (width 0.25) (layer "F.Cu") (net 5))
 (segment (start 102.235 76.6926) (end 102.6493 77.1069) (width 0.25) (layer "F.Cu") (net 5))
 (segment (start 103.1521 77.1069) (end 103.1521 77.107) (width 0.25) (layer "F.Cu") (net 5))
 (segment (start 108.37 89.3412) (end 108.89 88.8212) (width 0.25) (layer "F.Cu") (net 5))
 (segment (start 106.0836 84.6074) (end 106.0838 84.6076) (width 0.25) (layer "F.Cu") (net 5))
 (segment (start 106.0838 84.6076) (end 106.084 84.6074) (width 0.25) (layer "F.Cu") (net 5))
 (segment (start 102.6493 77.1069) (end 103.1521 77.1069) (width 0.25) (layer "F.Cu") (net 5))
 (segment (start 104.9374 86.5886) (end 104.7596 86.7664) (width 0.25) (layer "F.Cu") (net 5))
 (segment (start 104.9375 86.5886) (end 104.76 86.7664) (width 0.25) (layer "F.Cu") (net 5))
 (segment (start 105.115 86.4108) (end 105.115 85.5758) (width 0.25) (layer "F.Cu") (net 5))
 (segment (start 107.769 89.3412) (end 108.37 89.3412) (width 0.25) (layer "F.Cu") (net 5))
 (segment (start 105.115 86.4108) (end 104.9375 86.5886) (width 0.25) (layer "F.Cu") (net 5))
 (segment (start 107.769 89.3412) (end 107.7688 89.3412) (width 0.25) (layer "F.Cu") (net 5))
 (segment (start 104.9375 86.5886) (end 104.9374 86.5886) (width 0.25) (layer "F.Cu") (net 5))
 (via (at 103.1521 77.107) (size 0.8) (drill 0.4) (layers "F.Cu" "B.Cu") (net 5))
 (segment (start 99.3587 82.9434) (end 99.3587 80.9004) (width 0.25) (layer "B.Cu") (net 5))
 (segment (start 105.7565 89.3412) (end 99.3587 82.9434) (width 0.25) (layer "B.Cu") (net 5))
 (segment (start 99.3587 80.9004) (end 103.1521 77.107) (width 0.25) (layer "B.Cu") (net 5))
 (segment (start 107.7688 89.3412) (end 105.7565 89.3412) (width 0.25) (layer "B.Cu") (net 5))
 (segment (start 109.144 82.7024) (end 107.7082 82.7024) (width 0.25) (layer "F.Cu") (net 6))
 (segment (start 99.6596 89.3064) (end 100.922 90.5687) (width 0.25) (layer "F.Cu") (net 6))
 (segment (start 110.414 83.9724) (end 109.144 82.7024) (width 0.25) (layer "F.Cu") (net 6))
 (segment (start 110.414 90.4494) (end 110.414 83.9724) (width 0.25) (layer "F.Cu") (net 6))
 (segment (start 110.294 90.5687) (end 110.414 90.4494) (width 0.25) (layer "F.Cu") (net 6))
 (segment (start 107.7082 82.7024) (end 107.708 82.7024) (width 0.25) (layer "F.Cu") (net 6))
 (segment (start 100.922 90.5687) (end 110.294 90.5687) (width 0.25) (layer "F.Cu") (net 6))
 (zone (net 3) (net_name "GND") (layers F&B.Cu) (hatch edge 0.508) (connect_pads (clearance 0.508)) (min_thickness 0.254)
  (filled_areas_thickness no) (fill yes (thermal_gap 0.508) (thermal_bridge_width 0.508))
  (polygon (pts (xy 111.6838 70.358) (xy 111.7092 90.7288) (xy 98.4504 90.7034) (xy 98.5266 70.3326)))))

